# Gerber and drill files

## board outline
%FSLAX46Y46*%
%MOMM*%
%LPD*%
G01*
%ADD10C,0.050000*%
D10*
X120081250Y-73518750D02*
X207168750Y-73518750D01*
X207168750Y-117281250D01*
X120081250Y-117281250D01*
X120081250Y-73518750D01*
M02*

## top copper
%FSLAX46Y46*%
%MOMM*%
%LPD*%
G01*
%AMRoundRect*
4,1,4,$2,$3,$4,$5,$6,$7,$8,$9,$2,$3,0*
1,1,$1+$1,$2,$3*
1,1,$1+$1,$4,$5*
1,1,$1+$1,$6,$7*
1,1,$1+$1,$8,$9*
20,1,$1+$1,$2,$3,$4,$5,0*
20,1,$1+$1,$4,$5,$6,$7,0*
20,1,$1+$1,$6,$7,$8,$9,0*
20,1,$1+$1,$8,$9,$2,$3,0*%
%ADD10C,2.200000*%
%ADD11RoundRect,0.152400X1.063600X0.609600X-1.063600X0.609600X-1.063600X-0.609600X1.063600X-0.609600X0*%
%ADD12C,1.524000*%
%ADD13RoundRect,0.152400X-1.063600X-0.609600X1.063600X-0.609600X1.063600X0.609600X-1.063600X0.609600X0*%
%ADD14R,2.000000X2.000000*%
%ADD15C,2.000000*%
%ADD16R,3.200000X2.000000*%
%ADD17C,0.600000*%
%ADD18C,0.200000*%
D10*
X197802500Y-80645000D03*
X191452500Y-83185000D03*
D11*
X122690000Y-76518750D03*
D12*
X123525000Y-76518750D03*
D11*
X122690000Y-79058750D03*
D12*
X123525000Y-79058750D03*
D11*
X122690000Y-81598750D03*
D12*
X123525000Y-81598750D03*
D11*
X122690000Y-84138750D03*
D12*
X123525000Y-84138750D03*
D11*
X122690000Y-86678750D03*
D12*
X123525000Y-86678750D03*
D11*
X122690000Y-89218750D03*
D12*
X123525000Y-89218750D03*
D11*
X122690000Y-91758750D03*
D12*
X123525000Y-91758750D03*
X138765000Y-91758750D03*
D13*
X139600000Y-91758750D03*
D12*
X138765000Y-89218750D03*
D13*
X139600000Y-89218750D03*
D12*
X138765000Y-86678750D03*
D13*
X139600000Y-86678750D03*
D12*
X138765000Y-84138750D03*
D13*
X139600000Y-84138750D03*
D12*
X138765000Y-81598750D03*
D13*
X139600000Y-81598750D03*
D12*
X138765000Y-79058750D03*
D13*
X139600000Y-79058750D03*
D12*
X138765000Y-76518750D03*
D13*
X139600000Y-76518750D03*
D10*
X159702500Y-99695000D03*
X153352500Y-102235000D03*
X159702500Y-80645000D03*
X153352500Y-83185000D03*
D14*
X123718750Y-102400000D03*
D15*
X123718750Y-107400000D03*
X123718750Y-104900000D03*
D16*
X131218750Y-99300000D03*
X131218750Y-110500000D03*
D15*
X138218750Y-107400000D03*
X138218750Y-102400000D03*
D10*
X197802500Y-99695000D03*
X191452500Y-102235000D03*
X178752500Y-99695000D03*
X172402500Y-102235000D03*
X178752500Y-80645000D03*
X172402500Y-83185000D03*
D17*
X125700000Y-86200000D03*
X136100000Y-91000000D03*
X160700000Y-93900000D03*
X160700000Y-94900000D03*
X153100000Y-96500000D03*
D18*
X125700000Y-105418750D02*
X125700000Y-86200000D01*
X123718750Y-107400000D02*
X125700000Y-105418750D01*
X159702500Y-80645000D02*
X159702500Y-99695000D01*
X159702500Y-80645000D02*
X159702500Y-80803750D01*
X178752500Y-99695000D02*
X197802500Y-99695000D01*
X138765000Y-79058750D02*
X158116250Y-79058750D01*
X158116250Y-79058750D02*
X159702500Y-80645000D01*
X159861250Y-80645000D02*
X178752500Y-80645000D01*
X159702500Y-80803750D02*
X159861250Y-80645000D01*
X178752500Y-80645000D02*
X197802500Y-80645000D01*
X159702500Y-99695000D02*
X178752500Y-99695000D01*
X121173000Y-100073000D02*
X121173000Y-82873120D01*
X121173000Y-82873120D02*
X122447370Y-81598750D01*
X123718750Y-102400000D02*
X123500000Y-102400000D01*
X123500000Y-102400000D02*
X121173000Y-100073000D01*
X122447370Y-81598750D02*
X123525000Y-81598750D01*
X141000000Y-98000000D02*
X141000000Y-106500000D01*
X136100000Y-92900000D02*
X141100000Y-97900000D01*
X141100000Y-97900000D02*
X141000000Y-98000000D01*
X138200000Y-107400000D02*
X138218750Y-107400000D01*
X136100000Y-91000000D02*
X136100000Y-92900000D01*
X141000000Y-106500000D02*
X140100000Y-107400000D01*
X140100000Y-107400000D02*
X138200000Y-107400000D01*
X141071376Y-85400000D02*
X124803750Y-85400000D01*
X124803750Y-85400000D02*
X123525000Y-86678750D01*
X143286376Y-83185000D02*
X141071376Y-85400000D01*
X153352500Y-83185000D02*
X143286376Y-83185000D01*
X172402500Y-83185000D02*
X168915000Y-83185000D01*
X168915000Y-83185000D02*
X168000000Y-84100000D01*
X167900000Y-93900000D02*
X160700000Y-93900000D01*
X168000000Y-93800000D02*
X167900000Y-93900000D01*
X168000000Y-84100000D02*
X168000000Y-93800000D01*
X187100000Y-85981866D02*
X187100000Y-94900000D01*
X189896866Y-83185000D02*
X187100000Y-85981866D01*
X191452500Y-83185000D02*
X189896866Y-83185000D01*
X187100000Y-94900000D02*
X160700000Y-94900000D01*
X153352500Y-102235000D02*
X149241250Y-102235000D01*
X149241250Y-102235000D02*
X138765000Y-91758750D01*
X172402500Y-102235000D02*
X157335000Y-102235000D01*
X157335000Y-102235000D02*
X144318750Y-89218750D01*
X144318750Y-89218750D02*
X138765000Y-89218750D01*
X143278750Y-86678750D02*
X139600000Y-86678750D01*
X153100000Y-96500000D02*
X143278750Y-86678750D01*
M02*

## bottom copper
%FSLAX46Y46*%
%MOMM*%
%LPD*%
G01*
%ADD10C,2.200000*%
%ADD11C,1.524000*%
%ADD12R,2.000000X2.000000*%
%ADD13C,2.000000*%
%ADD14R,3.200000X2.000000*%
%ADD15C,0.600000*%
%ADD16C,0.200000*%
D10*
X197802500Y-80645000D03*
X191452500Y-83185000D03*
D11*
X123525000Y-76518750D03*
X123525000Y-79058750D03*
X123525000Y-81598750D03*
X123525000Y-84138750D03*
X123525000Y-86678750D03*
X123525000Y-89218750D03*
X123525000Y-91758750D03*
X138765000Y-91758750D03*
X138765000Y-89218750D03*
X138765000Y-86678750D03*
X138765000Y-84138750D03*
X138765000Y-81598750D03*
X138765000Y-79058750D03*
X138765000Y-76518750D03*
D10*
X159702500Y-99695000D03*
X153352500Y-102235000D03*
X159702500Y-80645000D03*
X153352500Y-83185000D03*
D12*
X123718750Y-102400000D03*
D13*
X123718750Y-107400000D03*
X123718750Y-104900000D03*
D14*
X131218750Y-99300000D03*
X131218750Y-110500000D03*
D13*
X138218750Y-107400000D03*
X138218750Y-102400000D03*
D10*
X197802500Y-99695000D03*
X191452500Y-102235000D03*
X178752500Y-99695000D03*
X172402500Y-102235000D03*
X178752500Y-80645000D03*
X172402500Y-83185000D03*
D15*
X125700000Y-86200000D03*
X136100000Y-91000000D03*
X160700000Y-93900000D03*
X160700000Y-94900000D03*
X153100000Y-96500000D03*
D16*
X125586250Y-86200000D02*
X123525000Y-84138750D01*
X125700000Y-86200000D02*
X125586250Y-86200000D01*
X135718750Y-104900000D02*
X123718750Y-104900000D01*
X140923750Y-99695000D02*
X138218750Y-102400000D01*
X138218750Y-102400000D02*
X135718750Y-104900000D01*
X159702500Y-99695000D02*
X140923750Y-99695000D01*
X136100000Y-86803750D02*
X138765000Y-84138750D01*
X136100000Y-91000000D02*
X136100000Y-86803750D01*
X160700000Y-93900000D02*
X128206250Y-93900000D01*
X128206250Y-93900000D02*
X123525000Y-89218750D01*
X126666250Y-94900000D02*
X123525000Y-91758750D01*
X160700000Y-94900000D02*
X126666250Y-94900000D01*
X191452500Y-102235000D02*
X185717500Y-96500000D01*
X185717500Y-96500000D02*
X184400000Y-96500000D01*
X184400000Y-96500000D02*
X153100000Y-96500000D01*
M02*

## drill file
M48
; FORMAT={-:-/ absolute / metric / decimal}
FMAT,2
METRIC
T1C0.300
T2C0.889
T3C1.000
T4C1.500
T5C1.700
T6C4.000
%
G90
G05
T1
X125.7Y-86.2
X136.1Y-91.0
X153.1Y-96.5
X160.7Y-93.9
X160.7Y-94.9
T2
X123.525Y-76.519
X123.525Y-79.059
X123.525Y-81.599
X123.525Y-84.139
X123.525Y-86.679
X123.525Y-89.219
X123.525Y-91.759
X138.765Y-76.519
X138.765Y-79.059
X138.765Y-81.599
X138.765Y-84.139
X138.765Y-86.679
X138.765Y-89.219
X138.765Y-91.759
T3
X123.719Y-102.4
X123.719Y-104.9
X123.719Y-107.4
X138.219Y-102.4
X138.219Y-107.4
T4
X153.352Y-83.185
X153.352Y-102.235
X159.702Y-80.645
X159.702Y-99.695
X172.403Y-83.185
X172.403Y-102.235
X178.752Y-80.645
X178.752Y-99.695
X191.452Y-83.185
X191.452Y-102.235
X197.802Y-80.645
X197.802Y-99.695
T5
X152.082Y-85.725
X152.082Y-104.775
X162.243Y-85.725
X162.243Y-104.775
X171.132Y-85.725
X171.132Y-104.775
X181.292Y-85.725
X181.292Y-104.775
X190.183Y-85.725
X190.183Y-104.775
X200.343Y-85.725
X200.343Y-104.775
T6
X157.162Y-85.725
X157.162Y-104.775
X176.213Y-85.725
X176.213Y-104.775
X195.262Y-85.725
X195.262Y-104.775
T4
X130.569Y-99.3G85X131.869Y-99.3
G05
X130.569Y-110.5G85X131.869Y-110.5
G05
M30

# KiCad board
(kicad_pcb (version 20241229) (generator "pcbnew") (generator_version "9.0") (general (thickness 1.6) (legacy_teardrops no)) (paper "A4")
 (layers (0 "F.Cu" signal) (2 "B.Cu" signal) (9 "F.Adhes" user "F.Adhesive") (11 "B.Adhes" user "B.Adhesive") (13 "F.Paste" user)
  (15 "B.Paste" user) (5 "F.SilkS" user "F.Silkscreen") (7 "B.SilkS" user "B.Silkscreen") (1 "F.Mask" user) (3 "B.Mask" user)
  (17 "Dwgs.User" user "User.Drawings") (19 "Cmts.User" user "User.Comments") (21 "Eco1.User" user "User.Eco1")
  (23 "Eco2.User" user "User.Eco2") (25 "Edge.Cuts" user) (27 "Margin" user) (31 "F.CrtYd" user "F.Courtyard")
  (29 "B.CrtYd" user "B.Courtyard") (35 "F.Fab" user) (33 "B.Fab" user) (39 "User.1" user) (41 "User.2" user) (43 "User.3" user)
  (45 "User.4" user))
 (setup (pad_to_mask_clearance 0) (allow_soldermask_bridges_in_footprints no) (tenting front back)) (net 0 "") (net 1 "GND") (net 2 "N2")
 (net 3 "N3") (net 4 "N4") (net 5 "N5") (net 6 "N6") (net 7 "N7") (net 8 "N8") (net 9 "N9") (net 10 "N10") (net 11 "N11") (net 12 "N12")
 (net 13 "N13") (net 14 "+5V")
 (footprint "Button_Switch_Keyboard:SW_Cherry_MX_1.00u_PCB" (layer "F.Cu") (at 197.8025 80.645)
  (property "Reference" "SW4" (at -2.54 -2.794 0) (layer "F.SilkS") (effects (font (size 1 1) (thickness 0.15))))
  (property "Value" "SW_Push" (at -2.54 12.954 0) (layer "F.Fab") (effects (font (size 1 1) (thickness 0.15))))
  (pad "" np_thru_hole circle (at -7.62 5.08) (size 1.7 1.7) (drill 1.7) (layers "*.Cu" "*.Mask"))
  (pad "" np_thru_hole circle (at -2.54 5.08) (size 4 4) (drill 4) (layers "*.Cu" "*.Mask"))
  (pad "" np_thru_hole circle (at 2.54 5.08) (size 1.7 1.7) (drill 1.7) (layers "*.Cu" "*.Mask"))
  (pad "1" thru_hole circle (at 0 0) (size 2.2 2.2) (drill 1.5) (layers "*.Cu" "*.Mask") (remove_unused_layers no) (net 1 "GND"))
  (pad "2" thru_hole circle (at -6.35 2.54) (size 2.2 2.2) (drill 1.5) (layers "*.Cu" "*.Mask") (remove_unused_layers no) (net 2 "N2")))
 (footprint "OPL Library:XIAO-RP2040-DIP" (layer "F.Cu") (at 131.145 84.13875)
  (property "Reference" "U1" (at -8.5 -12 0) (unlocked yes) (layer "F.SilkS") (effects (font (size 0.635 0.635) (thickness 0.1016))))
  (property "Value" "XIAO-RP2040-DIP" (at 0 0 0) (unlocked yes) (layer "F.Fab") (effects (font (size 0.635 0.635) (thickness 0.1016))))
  (pad "1" smd roundrect (at -8.455 -7.62 180) (size 2.432 1.524) (layers "F.Cu" "F.Mask") (roundrect_rratio 0.1) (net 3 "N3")
   (thermal_bridge_angle 45))
  (pad "1" thru_hole circle (at -7.62 -7.62 180) (size 1.524 1.524) (drill 0.889) (layers "*.Cu" "*.Mask") (remove_unused_layers no)
   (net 3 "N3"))
  (pad "2" smd roundrect (at -8.455 -5.08 180) (size 2.432 1.524) (layers "F.Cu" "F.Mask") (roundrect_rratio 0.1) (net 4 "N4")
   (thermal_bridge_angle 45))
  (pad "2" thru_hole circle (at -7.62 -5.08 180) (size 1.524 1.524) (drill 0.889) (layers "*.Cu" "*.Mask") (remove_unused_layers no)
   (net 4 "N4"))
  (pad "3" smd roundrect (at -8.455 -2.54 180) (size 2.432 1.524) (layers "F.Cu" "F.Mask") (roundrect_rratio 0.1) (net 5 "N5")
   (thermal_bridge_angle 45))
  (pad "3" thru_hole circle (at -7.62 -2.54 180) (size 1.524 1.524) (drill 0.889) (layers "*.Cu" "*.Mask") (remove_unused_layers no)
   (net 5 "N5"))
  (pad "4" smd roundrect (at -8.455 0 180) (size 2.432 1.524) (layers "F.Cu" "F.Mask") (roundrect_rratio 0.1) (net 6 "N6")
   (thermal_bridge_angle 45))
  (pad "4" thru_hole circle (at -7.62 0 180) (size 1.524 1.524) (drill 0.889) (layers "*.Cu" "*.Mask") (remove_unused_layers no)
   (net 6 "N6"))
  (pad "5" smd roundrect (at -8.455 2.54 180) (size 2.432 1.524) (layers "F.Cu" "F.Mask") (roundrect_rratio 0.1) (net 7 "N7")
   (thermal_bridge_angle 45))
  (pad "5" thru_hole circle (at -7.62 2.54 180) (size 1.524 1.524) (drill 0.889) (layers "*.Cu" "*.Mask") (remove_unused_layers no)
   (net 7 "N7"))
  (pad "6" smd roundrect (at -8.455 5.08 180) (size 2.432 1.524) (layers "F.Cu" "F.Mask") (roundrect_rratio 0.1) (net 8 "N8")
   (thermal_bridge_angle 45))
  (pad "6" thru_hole circle (at -7.62 5.08 180) (size 1.524 1.524) (drill 0.889) (layers "*.Cu" "*.Mask") (remove_unused_layers no)
   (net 8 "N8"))
  (pad "7" smd roundrect (at -8.455 7.62 180) (size 2.432 1.524) (layers "F.Cu" "F.Mask") (roundrect_rratio 0.1) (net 2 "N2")
   (thermal_bridge_angle 45))
  (pad "7" thru_hole circle (at -7.62 7.62 180) (size 1.524 1.524) (drill 0.889) (layers "*.Cu" "*.Mask") (remove_unused_layers no)
   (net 2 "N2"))
  (pad "8" thru_hole circle (at 7.62 7.62) (size 1.524 1.524) (drill 0.889) (layers "*.Cu" "*.Mask") (remove_unused_layers no) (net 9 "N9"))
  (pad "8" smd roundrect (at 8.455 7.62) (size 2.432 1.524) (layers "F.Cu" "F.Mask") (roundrect_rratio 0.1) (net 9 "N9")
   (thermal_bridge_angle 45))
  (pad "9" thru_hole circle (at 7.62 5.08) (size 1.524 1.524) (drill 0.889) (layers "*.Cu" "*.Mask") (remove_unused_layers no)
   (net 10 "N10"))
  (pad "9" smd roundrect (at 8.455 5.08) (size 2.432 1.524) (layers "F.Cu" "F.Mask") (roundrect_rratio 0.1) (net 10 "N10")
   (thermal_bridge_angle 45))
  (pad "10" thru_hole circle (at 7.62 2.54) (size 1.524 1.524) (drill 0.889) (layers "*.Cu" "*.Mask") (remove_unused_layers no)
   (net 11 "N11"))
  (pad "10" smd roundrect (at 8.455 2.54) (size 2.432 1.524) (layers "F.Cu" "F.Mask") (roundrect_rratio 0.1) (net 11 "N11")
   (thermal_bridge_angle 45))
  (pad "11" thru_hole circle (at 7.62 0) (size 1.524 1.524) (drill 0.889) (layers "*.Cu" "*.Mask") (remove_unused_layers no) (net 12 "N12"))
  (pad "11" smd roundrect (at 8.455 0) (size 2.432 1.524) (layers "F.Cu" "F.Mask") (roundrect_rratio 0.1) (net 12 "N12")
   (thermal_bridge_angle 45))
  (pad "12" thru_hole circle (at 7.62 -2.54) (size 1.524 1.524) (drill 0.889) (layers "*.Cu" "*.Mask") (remove_unused_layers no)
   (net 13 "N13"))
  (pad "12" smd roundrect (at 8.455 -2.54) (size 2.432 1.524) (layers "F.Cu" "F.Mask") (roundrect_rratio 0.1) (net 13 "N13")
   (thermal_bridge_angle 45))
  (pad "13" thru_hole circle (at 7.62 -5.08) (size 1.524 1.524) (drill 0.889) (layers "*.Cu" "*.Mask") (remove_unused_layers no)
   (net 1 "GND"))
  (pad "13" smd roundrect (at 8.455 -5.08) (size 2.432 1.524) (layers "F.Cu" "F.Mask") (roundrect_rratio 0.1) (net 1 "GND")
   (thermal_bridge_angle 45))
  (pad "14" thru_hole circle (at 7.62 -7.62) (size 1.524 1.524) (drill 0.889) (layers "*.Cu" "*.Mask") (remove_unused_layers no)
   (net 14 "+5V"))
  (pad "14" smd roundrect (at 8.455 -7.62) (size 2.432 1.524) (layers "F.Cu" "F.Mask") (roundrect_rratio 0.1) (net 14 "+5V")
   (thermal_bridge_angle 45)))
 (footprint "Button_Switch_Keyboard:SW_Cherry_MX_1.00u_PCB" (layer "F.Cu") (at 159.7025 99.695)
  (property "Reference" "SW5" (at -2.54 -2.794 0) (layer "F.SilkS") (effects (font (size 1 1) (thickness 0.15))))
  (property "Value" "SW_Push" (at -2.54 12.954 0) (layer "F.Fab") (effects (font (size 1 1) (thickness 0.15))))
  (pad "" np_thru_hole circle (at -7.62 5.08) (size 1.7 1.7) (drill 1.7) (layers "*.Cu" "*.Mask"))
  (pad "" np_thru_hole circle (at -2.54 5.08) (size 4 4) (drill 4) (layers "*.Cu" "*.Mask"))
  (pad "" np_thru_hole circle (at 2.54 5.08) (size 1.7 1.7) (drill 1.7) (layers "*.Cu" "*.Mask"))
  (pad "1" thru_hole circle (at 0 0) (size 2.2 2.2) (drill 1.5) (layers "*.Cu" "*.Mask") (remove_unused_layers no) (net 1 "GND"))
  (pad "2" thru_hole circle (at -6.35 2.54) (size 2.2 2.2) (drill 1.5) (layers "*.Cu" "*.Mask") (remove_unused_layers no) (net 9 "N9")))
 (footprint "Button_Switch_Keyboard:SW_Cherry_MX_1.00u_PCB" (layer "F.Cu") (at 159.7025 80.645)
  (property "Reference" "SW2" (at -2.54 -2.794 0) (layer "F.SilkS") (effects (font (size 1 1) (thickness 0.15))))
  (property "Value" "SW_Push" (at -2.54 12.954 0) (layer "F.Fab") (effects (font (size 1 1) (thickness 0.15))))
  (pad "" np_thru_hole circle (at -7.62 5.08) (size 1.7 1.7) (drill 1.7) (layers "*.Cu" "*.Mask"))
  (pad "" np_thru_hole circle (at -2.54 5.08) (size 4 4) (drill 4) (layers "*.Cu" "*.Mask"))
  (pad "" np_thru_hole circle (at 2.54 5.08) (size 1.7 1.7) (drill 1.7) (layers "*.Cu" "*.Mask"))
  (pad "1" thru_hole circle (at 0 0) (size 2.2 2.2) (drill 1.5) (layers "*.Cu" "*.Mask") (remove_unused_layers no) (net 1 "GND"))
  (pad "2" thru_hole circle (at -6.35 2.54) (size 2.2 2.2) (drill 1.5) (layers "*.Cu" "*.Mask") (remove_unused_layers no) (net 7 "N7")))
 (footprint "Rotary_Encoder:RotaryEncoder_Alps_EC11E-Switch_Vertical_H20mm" (layer "F.Cu") (at 123.71875 102.4)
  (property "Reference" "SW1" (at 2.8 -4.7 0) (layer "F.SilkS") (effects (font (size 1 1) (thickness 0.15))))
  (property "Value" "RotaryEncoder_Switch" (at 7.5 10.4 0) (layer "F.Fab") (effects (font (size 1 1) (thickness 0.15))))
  (pad "A" thru_hole rect (at 0 0) (size 2 2) (drill 1) (layers "*.Cu" "*.Mask") (remove_unused_layers no) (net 5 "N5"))
  (pad "B" thru_hole circle (at 0 5) (size 2 2) (drill 1) (layers "*.Cu" "*.Mask") (remove_unused_layers no) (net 6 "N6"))
  (pad "C" thru_hole circle (at 0 2.5) (size 2 2) (drill 1) (layers "*.Cu" "*.Mask") (remove_unused_layers no) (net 1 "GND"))
  (pad "MP" thru_hole rect (at 7.5 -3.1) (size 3.2 2) (drill oval 2.8 1.5) (layers "*.Cu" "*.Mask") (remove_unused_layers no))
  (pad "MP" thru_hole rect (at 7.5 8.1) (size 3.2 2) (drill oval 2.8 1.5) (layers "*.Cu" "*.Mask") (remove_unused_layers no))
  (pad "S1" thru_hole circle (at 14.5 5) (size 2 2) (drill 1) (layers "*.Cu" "*.Mask") (remove_unused_layers no) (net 12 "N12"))
  (pad "S2" thru_hole circle (at 14.5 0) (size 2 2) (drill 1) (layers "*.Cu" "*.Mask") (remove_unused_layers no) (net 1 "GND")))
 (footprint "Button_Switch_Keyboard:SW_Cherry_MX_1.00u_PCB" (layer "F.Cu") (at 197.8025 99.695)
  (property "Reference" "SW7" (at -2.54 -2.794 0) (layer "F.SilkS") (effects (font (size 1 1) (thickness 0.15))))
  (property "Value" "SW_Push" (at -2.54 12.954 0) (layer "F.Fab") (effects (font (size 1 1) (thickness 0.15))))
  (pad "" np_thru_hole circle (at -7.62 5.08) (size 1.7 1.7) (drill 1.7) (layers "*.Cu" "*.Mask"))
  (pad "" np_thru_hole circle (at -2.54 5.08) (size 4 4) (drill 4) (layers "*.Cu" "*.Mask"))
  (pad "" np_thru_hole circle (at 2.54 5.08) (size 1.7 1.7) (drill 1.7) (layers "*.Cu" "*.Mask"))
  (pad "1" thru_hole circle (at 0 0) (size 2.2 2.2) (drill 1.5) (layers "*.Cu" "*.Mask") (remove_unused_layers no) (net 1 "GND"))
  (pad "2" thru_hole circle (at -6.35 2.54) (size 2.2 2.2) (drill 1.5) (layers "*.Cu" "*.Mask") (remove_unused_layers no) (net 11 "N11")))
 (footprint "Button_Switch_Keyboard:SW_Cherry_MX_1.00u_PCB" (layer "F.Cu") (at 178.7525 99.695)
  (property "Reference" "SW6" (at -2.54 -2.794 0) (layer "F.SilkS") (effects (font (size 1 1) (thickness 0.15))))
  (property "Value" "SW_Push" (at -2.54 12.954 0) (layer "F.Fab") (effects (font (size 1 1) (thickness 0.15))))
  (pad "" np_thru_hole circle (at -7.62 5.08) (size 1.7 1.7) (drill 1.7) (layers "*.Cu" "*.Mask"))
  (pad "" np_thru_hole circle (at -2.54 5.08) (size 4 4) (drill 4) (layers "*.Cu" "*.Mask"))
  (pad "" np_thru_hole circle (at 2.54 5.08) (size 1.7 1.7) (drill 1.7) (layers "*.Cu" "*.Mask"))
  (pad "1" thru_hole circle (at 0 0) (size 2.2 2.2) (drill 1.5) (layers "*.Cu" "*.Mask") (remove_unused_layers no) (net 1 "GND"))
  (pad "2" thru_hole circle (at -6.35 2.54) (size 2.2 2.2) (drill 1.5) (layers "*.Cu" "*.Mask") (remove_unused_layers no) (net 10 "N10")))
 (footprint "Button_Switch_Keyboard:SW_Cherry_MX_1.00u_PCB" (layer "F.Cu") (at 178.7525 80.645)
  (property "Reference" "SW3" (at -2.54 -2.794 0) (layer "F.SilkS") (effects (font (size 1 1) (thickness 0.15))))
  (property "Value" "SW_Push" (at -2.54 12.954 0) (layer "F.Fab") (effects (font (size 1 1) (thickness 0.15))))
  (pad "" np_thru_hole circle (at -7.62 5.08) (size 1.7 1.7) (drill 1.7) (layers "*.Cu" "*.Mask"))
  (pad "" np_thru_hole circle (at -2.54 5.08) (size 4 4) (drill 4) (layers "*.Cu" "*.Mask"))
  (pad "" np_thru_hole circle (at 2.54 5.08) (size 1.7 1.7) (drill 1.7) (layers "*.Cu" "*.Mask"))
  (pad "1" thru_hole circle (at 0 0) (size 2.2 2.2) (drill 1.5) (layers "*.Cu" "*.Mask") (remove_unused_layers no) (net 1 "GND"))
  (pad "2" thru_hole circle (at -6.35 2.54) (size 2.2 2.2) (drill 1.5) (layers "*.Cu" "*.Mask") (remove_unused_layers no) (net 8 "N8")))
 (gr_rect (start 120.08125 73.51875) (end 207.16875 117.28125) (stroke (width 0.05) (type default)) (fill no) (layer "Edge.Cuts"))
 (segment (start 125.7 105.41875) (end 125.7 86.2) (width 0.2) (layer "F.Cu") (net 6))
 (segment (start 123.71875 107.4) (end 125.7 105.41875) (width 0.2) (layer "F.Cu") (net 6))
 (via (at 125.7 86.2) (size 0.6) (drill 0.3) (layers "F.Cu" "B.Cu") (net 6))
 (segment (start 125.58625 86.2) (end 123.525 84.13875) (width 0.2) (layer "B.Cu") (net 6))
 (segment (start 125.7 86.2) (end 125.58625 86.2) (width 0.2) (layer "B.Cu") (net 6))
 (segment (start 159.7025 80.645) (end 159.7025 99.695) (width 0.2) (layer "F.Cu") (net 1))
 (segment (start 159.7025 80.645) (end 159.7025 80.80375) (width 0.2) (layer "F.Cu") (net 1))
 (segment (start 178.7525 99.695) (end 197.8025 99.695) (width 0.2) (layer "F.Cu") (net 1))
 (segment (start 138.765 79.05875) (end 158.11625 79.05875) (width 0.2) (layer "F.Cu") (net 1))
 (segment (start 158.11625 79.05875) (end 159.7025 80.645) (width 0.2) (layer "F.Cu") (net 1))
 (segment (start 159.86125 80.645) (end 178.7525 80.645) (width 0.2) (layer "F.Cu") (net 1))
 (segment (start 159.7025 80.80375) (end 159.86125 80.645) (width 0.2) (layer "F.Cu") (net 1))
 (segment (start 178.7525 80.645) (end 197.8025 80.645) (width 0.2) (layer "F.Cu") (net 1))
 (segment (start 159.7025 99.695) (end 178.7525 99.695) (width 0.2) (layer "F.Cu") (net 1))
 (segment (start 135.71875 104.9) (end 123.71875 104.9) (width 0.2) (layer "B.Cu") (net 1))
 (segment (start 140.92375 99.695) (end 138.21875 102.4) (width 0.2) (layer "B.Cu") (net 1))
 (segment (start 138.21875 102.4) (end 135.71875 104.9) (width 0.2) (layer "B.Cu") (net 1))
 (segment (start 159.7025 99.695) (end 140.92375 99.695) (width 0.2) (layer "B.Cu") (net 1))
 (segment (start 121.173 100.073) (end 121.173 82.87312) (width 0.2) (layer "F.Cu") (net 5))
 (segment (start 121.173 82.87312) (end 122.44737 81.59875) (width 0.2) (layer "F.Cu") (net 5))
 (segment (start 123.71875 102.4) (end 123.5 102.4) (width 0.2) (layer "F.Cu") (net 5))
 (segment (start 123.5 102.4) (end 121.173 100.073) (width 0.2) (layer "F.Cu") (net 5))
 (segment (start 122.44737 81.59875) (end 123.525 81.59875) (width 0.2) (layer "F.Cu") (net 5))
 (segment (start 141 98) (end 141 106.5) (width 0.2) (layer "F.Cu") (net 12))
 (segment (start 136.1 92.9) (end 141.1 97.9) (width 0.2) (layer "F.Cu") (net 12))
 (segment (start 141.1 97.9) (end 141 98) (width 0.2) (layer "F.Cu") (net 12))
 (segment (start 138.2 107.4) (end 138.21875 107.4) (width 0.2) (layer "F.Cu") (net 12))
 (segment (start 136.1 91) (end 136.1 92.9) (width 0.2) (layer "F.Cu") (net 12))
 (segment (start 141 106.5) (end 140.1 107.4) (width 0.2) (layer "F.Cu") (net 12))
 (segment (start 140.1 107.4) (end 138.2 107.4) (width 0.2) (layer "F.Cu") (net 12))
 (via (at 136.1 91) (size 0.6) (drill 0.3) (layers "F.Cu" "B.Cu") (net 12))
 (segment (start 136.1 86.80375) (end 138.765 84.13875) (width 0.2) (layer "B.Cu") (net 12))
 (segment (start 136.1 91) (end 136.1 86.80375) (width 0.2) (layer "B.Cu") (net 12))
 (segment (start 141.071376 85.4) (end 124.80375 85.4) (width 0.2) (layer "F.Cu") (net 7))
 (segment (start 124.80375 85.4) (end 123.525 86.67875) (width 0.2) (layer "F.Cu") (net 7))
 (segment (start 143.286376 83.185) (end 141.071376 85.4) (width 0.2) (layer "F.Cu") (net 7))
 (segment (start 153.3525 83.185) (end 143.286376 83.185) (width 0.2) (layer "F.Cu") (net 7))
 (segment (start 172.4025 83.185) (end 168.915 83.185) (width 0.2) (layer "F.Cu") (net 8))
 (segment (start 168.915 83.185) (end 168 84.1) (width 0.2) (layer "F.Cu") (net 8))
 (segment (start 167.9 93.9) (end 160.7 93.9) (width 0.2) (layer "F.Cu") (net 8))
 (segment (start 168 93.8) (end 167.9 93.9) (width 0.2) (layer "F.Cu") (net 8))
 (segment (start 168 84.1) (end 168 93.8) (width 0.2) (layer "F.Cu") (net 8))
 (via (at 160.7 93.9) (size 0.6) (drill 0.3) (layers "F.Cu" "B.Cu") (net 8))
 (segment (start 160.7 93.9) (end 128.20625 93.9) (width 0.2) (layer "B.Cu") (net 8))
 (segment (start 128.20625 93.9) (end 123.525 89.21875) (width 0.2) (layer "B.Cu") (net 8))
 (segment (start 187.1 85.981866) (end 187.1 94.9) (width 0.2) (layer "F.Cu") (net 2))
 (segment (start 189.896866 83.185) (end 187.1 85.981866) (width 0.2) (layer "F.Cu") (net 2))
 (segment (start 191.4525 83.185) (end 189.896866 83.185) (width 0.2) (layer "F.Cu") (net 2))
 (segment (start 187.1 94.9) (end 160.7 94.9) (width 0.2) (layer "F.Cu") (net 2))
 (via (at 160.7 94.9) (size 0.6) (drill 0.3) (layers "F.Cu" "B.Cu") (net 2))
 (segment (start 126.66625 94.9) (end 123.525 91.75875) (width 0.2) (layer "B.Cu") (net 2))
 (segment (start 160.7 94.9) (end 126.66625 94.9) (width 0.2) (layer "B.Cu") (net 2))
 (segment (start 153.3525 102.235) (end 149.24125 102.235) (width 0.2) (layer "F.Cu") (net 9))
 (segment (start 149.24125 102.235) (end 138.765 91.75875) (width 0.2) (layer "F.Cu") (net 9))
 (segment (start 172.4025 102.235) (end 157.335 102.235) (width 0.2) (layer "F.Cu") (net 10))
 (segment (start 157.335 102.235) (end 144.31875 89.21875) (width 0.2) (layer "F.Cu") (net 10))
 (segment (start 144.31875 89.21875) (end 138.765 89.21875) (width 0.2) (layer "F.Cu") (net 10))
 (segment (start 143.27875 86.67875) (end 139.6 86.67875) (width 0.2) (layer "F.Cu") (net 11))
 (segment (start 153.1 96.5) (end 143.27875 86.67875) (width 0.2) (layer "F.Cu") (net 11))
 (via (at 153.1 96.5) (size 0.6) (drill 0.3) (layers "F.Cu" "B.Cu") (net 11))
 (segment (start 191.4525 102.235) (end 185.7175 96.5) (width 0.2) (layer "B.Cu") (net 11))
 (segment (start 185.7175 96.5) (end 184.4 96.5) (width 0.2) (layer "B.Cu") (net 11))
 (segment (start 184.4 96.5) (end 153.1 96.5) (width 0.2) (layer "B.Cu") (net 11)))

